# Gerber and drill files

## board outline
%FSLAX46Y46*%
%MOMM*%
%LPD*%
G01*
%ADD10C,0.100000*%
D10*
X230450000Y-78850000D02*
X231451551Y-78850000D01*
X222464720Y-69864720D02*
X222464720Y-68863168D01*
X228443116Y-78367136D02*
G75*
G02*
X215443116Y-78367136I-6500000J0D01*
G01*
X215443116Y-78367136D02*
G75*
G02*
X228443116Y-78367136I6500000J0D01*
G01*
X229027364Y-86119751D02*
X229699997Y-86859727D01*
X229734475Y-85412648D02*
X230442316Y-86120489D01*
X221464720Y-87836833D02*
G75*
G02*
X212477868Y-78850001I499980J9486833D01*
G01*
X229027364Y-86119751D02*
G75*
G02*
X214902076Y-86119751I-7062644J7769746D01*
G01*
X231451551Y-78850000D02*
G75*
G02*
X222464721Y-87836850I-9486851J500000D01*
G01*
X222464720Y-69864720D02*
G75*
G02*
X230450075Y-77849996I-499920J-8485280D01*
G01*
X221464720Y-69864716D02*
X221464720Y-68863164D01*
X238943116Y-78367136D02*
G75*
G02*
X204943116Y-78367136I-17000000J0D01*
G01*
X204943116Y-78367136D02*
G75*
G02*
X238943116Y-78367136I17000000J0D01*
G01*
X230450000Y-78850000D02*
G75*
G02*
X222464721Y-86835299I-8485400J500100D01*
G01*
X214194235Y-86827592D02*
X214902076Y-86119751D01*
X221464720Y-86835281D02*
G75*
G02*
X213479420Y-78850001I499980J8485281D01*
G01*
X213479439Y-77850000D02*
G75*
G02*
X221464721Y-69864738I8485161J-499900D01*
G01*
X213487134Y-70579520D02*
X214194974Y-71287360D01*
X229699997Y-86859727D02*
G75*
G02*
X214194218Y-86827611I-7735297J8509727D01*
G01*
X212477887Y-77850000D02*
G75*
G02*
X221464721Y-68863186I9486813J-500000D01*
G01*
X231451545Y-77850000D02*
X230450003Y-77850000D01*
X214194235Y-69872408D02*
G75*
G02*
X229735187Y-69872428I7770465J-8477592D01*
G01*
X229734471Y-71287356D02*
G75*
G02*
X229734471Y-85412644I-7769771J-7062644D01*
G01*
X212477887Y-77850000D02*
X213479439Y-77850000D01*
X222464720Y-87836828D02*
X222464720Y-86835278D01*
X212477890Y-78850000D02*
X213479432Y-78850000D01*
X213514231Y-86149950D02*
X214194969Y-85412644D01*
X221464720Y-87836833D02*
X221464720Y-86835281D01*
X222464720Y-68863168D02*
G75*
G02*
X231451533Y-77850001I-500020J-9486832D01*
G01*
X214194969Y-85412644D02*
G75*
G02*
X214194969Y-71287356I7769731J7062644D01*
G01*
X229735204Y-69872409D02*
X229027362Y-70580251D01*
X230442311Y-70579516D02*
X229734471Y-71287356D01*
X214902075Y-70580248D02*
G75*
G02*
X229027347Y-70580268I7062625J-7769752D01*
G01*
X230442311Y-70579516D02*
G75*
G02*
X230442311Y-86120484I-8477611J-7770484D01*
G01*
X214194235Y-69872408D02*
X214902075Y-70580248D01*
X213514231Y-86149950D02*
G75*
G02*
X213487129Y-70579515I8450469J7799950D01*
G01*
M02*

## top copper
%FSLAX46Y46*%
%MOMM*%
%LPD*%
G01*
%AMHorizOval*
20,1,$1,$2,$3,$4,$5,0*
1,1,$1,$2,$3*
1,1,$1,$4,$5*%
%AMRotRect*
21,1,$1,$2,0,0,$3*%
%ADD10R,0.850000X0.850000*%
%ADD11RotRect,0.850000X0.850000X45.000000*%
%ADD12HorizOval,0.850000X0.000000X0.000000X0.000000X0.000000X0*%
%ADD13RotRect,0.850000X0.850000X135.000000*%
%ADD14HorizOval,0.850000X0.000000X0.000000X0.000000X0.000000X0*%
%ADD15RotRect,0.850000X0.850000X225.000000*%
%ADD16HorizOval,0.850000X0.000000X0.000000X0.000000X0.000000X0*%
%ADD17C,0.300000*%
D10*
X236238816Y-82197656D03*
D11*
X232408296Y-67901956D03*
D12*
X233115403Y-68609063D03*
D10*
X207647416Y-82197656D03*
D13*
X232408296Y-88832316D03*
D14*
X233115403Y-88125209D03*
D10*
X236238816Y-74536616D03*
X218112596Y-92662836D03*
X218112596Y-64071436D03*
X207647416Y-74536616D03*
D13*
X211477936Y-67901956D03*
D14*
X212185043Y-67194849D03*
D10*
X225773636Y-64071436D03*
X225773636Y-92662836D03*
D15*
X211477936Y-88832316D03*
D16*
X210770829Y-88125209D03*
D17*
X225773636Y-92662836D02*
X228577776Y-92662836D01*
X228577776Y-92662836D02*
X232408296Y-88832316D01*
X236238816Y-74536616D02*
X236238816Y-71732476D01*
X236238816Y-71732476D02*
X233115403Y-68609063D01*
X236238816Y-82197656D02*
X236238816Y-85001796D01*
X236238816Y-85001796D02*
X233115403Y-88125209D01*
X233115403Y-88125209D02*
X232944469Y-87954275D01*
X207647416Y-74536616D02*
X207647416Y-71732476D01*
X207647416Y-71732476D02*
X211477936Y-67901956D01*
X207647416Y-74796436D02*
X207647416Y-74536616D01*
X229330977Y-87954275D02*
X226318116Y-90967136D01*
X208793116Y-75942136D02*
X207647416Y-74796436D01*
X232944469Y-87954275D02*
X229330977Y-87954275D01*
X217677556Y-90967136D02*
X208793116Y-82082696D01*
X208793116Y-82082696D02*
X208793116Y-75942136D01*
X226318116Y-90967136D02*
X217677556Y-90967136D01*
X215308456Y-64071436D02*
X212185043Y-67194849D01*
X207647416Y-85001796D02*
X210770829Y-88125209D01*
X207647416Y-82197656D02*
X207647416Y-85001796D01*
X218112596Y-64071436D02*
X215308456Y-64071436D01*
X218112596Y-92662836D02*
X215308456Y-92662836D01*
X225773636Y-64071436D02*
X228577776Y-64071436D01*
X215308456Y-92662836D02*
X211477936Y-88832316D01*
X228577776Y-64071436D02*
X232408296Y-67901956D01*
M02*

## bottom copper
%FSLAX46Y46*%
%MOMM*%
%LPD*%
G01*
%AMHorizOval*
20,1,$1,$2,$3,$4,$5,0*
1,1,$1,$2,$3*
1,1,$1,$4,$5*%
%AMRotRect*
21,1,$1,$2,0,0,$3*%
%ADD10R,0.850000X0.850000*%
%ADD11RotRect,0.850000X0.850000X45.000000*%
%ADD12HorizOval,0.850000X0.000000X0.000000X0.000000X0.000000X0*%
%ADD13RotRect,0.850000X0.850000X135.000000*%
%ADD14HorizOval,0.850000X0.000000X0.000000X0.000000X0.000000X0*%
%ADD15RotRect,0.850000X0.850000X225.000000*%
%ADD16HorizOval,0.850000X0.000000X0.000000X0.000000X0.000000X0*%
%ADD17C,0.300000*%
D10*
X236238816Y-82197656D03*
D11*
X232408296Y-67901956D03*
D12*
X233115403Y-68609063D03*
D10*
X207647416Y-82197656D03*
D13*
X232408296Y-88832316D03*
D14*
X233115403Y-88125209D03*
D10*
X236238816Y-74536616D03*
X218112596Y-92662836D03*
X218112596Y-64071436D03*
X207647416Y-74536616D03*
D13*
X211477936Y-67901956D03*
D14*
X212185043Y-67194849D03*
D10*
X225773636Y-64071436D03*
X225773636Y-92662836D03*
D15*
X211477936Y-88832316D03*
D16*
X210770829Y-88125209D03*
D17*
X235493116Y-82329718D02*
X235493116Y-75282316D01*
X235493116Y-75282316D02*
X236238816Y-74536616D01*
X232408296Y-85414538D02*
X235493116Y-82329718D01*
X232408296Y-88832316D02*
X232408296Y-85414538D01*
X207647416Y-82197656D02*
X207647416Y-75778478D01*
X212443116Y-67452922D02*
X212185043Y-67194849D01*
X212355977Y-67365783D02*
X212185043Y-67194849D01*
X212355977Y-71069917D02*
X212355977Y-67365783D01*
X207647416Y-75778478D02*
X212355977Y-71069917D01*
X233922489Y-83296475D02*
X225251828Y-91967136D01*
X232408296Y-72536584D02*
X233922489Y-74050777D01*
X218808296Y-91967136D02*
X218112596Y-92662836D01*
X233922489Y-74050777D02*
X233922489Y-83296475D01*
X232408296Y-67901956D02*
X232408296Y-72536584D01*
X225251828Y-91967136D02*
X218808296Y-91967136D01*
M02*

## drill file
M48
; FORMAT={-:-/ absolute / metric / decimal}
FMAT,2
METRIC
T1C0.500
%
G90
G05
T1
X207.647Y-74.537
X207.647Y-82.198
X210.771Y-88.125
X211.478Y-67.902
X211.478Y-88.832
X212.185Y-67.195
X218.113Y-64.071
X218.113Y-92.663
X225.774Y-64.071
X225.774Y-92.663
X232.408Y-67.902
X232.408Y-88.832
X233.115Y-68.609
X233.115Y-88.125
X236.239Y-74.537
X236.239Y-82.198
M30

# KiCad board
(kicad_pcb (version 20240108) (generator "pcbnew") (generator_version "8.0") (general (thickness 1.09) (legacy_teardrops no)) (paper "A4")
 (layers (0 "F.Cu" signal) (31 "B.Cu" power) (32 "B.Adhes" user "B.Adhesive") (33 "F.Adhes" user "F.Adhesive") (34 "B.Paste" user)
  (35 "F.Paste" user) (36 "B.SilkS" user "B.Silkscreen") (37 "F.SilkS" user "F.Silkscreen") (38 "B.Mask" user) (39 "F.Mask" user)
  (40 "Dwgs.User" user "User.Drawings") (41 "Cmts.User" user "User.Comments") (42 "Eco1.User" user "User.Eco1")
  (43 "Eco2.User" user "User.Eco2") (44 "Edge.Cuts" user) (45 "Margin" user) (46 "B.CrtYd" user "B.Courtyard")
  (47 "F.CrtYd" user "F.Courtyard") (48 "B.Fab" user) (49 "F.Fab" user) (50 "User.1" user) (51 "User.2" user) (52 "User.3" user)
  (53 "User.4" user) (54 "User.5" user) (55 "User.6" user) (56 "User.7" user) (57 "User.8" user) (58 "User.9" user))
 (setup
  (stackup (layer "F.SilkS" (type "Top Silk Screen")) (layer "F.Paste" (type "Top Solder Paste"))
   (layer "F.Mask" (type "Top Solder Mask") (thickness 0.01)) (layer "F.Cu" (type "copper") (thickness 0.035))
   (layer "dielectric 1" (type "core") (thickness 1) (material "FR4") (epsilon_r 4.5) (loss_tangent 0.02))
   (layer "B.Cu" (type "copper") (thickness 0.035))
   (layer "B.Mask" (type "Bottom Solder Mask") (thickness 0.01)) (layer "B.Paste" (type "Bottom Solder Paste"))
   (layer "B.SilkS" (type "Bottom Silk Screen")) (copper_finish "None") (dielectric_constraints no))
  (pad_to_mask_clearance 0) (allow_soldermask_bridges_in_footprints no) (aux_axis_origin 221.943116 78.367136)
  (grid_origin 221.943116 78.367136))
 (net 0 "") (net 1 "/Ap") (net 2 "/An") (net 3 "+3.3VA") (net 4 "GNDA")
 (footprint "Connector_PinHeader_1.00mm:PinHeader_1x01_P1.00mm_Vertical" (layer "F.Cu") (at 236.238816 82.197656)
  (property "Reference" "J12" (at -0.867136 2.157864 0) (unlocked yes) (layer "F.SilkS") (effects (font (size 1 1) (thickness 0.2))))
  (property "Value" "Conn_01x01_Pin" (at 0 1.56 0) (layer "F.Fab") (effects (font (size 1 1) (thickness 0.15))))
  (pad "1" thru_hole rect (at 0 0) (size 0.85 0.85) (drill 0.5) (layers "*.Cu" "*.Mask") (remove_unused_layers no) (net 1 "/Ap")))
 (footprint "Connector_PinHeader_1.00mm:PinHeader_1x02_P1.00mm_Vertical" (layer "F.Cu") (at 232.408296 67.901956 45)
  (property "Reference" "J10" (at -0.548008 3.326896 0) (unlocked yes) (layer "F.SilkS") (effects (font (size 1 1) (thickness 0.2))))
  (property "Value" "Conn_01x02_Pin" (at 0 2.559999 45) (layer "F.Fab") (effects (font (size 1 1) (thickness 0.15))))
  (pad "1" thru_hole rect (at 0 0 45) (size 0.85 0.85) (drill 0.5) (layers "*.Cu" "*.Mask") (remove_unused_layers no) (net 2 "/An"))
  (pad "2" thru_hole oval (at 0 1 45) (size 0.85 0.85) (drill 0.5) (layers "*.Cu" "*.Mask") (remove_unused_layers no) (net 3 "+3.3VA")))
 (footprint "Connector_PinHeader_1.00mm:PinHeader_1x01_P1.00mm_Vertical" (layer "F.Cu") (at 207.647416 82.197656)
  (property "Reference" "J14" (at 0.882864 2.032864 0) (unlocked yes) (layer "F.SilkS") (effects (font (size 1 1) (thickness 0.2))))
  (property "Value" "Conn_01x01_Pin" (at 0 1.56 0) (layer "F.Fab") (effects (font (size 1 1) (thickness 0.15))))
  (pad "1" thru_hole rect (at 0 0) (size 0.85 0.85) (drill 0.5) (layers "*.Cu" "*.Mask") (remove_unused_layers no) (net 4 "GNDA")))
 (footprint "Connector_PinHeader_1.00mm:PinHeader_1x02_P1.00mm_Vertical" (layer "F.Cu") (at 232.408296 88.832316 135)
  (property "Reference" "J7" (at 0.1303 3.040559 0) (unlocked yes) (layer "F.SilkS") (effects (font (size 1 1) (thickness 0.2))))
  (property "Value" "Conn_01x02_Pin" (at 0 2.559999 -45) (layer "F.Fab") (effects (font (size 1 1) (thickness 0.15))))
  (pad "1" thru_hole rect (at 0 0 135) (size 0.85 0.85) (drill 0.5) (layers "*.Cu" "*.Mask") (remove_unused_layers no) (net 3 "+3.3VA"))
  (pad "2" thru_hole oval (at 0 1 135) (size 0.85 0.85) (drill 0.5) (layers "*.Cu" "*.Mask") (remove_unused_layers no) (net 1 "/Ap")))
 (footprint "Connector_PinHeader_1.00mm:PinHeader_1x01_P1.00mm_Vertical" (layer "F.Cu") (at 236.238816 74.536616)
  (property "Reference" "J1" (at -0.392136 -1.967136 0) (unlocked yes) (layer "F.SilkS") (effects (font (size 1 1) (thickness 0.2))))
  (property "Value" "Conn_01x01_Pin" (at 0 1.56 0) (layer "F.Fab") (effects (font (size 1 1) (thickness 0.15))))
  (pad "1" thru_hole rect (at 0 0) (size 0.85 0.85) (drill 0.5) (layers "*.Cu" "*.Mask") (remove_unused_layers no) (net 3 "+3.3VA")))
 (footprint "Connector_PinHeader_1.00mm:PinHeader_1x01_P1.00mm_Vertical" (layer "F.Cu") (at 218.112596 92.662836)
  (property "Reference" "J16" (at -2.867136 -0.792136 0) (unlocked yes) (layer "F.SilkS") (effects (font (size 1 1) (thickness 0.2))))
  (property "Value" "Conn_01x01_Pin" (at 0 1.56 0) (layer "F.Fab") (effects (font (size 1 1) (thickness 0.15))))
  (pad "1" thru_hole rect (at 0 0) (size 0.85 0.85) (drill 0.5) (layers "*.Cu" "*.Mask") (remove_unused_layers no) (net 2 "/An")))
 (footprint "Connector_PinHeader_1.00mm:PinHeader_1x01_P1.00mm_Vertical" (layer "F.Cu") (at 218.112596 64.071436)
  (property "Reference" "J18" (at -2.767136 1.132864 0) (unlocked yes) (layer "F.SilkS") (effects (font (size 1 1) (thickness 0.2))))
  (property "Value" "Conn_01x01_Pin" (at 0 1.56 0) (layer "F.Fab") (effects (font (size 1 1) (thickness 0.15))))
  (pad "1" thru_hole rect (at 0 0) (size 0.85 0.85) (drill 0.5) (layers "*.Cu" "*.Mask") (remove_unused_layers no) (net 4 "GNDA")))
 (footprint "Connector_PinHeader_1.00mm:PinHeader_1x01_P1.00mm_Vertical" (layer "F.Cu") (at 207.647416 74.536616)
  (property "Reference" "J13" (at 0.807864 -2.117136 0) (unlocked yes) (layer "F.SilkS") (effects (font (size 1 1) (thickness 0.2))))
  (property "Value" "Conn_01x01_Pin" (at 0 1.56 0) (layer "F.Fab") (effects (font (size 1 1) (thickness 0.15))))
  (pad "1" thru_hole rect (at 0 0) (size 0.85 0.85) (drill 0.5) (layers "*.Cu" "*.Mask") (remove_unused_layers no) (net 1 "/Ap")))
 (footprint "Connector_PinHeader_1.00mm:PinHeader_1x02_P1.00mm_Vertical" (layer "F.Cu") (at 211.477936 67.901956 135)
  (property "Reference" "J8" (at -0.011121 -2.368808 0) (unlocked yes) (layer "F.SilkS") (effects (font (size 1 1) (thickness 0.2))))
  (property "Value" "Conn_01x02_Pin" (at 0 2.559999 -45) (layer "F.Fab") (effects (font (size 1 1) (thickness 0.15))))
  (pad "1" thru_hole rect (at 0 0 135) (size 0.85 0.85) (drill 0.5) (layers "*.Cu" "*.Mask") (remove_unused_layers no) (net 1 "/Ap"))
  (pad "2" thru_hole oval (at 0 1 135) (size 0.85 0.85) (drill 0.5) (layers "*.Cu" "*.Mask") (remove_unused_layers no) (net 4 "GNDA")))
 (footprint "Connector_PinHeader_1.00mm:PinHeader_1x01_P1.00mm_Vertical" (layer "F.Cu") (at 225.773636 64.071436)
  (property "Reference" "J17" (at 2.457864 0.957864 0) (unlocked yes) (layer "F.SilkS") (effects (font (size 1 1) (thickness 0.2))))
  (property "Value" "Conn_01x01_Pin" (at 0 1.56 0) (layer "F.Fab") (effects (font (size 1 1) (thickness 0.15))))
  (pad "1" thru_hole rect (at 0 0) (size 0.85 0.85) (drill 0.5) (layers "*.Cu" "*.Mask") (remove_unused_layers no) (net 2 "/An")))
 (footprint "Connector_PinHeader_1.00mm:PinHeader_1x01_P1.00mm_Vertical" (layer "F.Cu") (at 225.773636 92.662836)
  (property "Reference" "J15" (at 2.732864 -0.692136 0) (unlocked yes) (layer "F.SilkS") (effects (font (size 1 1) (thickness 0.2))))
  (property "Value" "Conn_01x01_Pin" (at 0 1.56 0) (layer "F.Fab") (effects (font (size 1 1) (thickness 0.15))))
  (pad "1" thru_hole rect (at 0 0) (size 0.85 0.85) (drill 0.5) (layers "*.Cu" "*.Mask") (remove_unused_layers no) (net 3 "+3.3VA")))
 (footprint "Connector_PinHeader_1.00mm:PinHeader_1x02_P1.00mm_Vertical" (layer "F.Cu") (at 211.477936 88.832316 -135)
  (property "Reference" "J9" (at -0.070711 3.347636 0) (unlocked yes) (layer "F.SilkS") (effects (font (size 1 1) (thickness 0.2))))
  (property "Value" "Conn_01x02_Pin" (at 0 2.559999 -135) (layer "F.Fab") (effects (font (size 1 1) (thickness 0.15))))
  (pad "1" thru_hole rect (at 0 0 225) (size 0.85 0.85) (drill 0.5) (layers "*.Cu" "*.Mask") (remove_unused_layers no) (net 2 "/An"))
  (pad "2" thru_hole oval (at 0 1 225) (size 0.85 0.85) (drill 0.5) (layers "*.Cu" "*.Mask") (remove_unused_layers no) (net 4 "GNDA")))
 (gr_line (start 230.45 78.85) (end 231.451551 78.85) (stroke (width 0.1) (type default)) (layer "Edge.Cuts"))
 (gr_line (start 222.46472 69.86472) (end 222.46472 68.863168) (stroke (width 0.1) (type default)) (layer "Edge.Cuts"))
 (gr_circle (center 221.943116 78.367136) (end 228.443116 78.367136) (stroke (width 0.1) (type default)) (fill none) (layer "Edge.Cuts"))
 (gr_line (start 229.027364 86.119751) (end 229.699997 86.859727) (stroke (width 0.1) (type default)) (layer "Edge.Cuts"))
 (gr_line (start 229.734475 85.412648) (end 230.442316 86.120489) (stroke (width 0.1) (type default)) (layer "Edge.Cuts"))
 (gr_arc (start 221.46472 87.836833) (mid 215.247206 85.067515) (end 212.47789 78.85) (stroke (width 0.1) (type default))
  (layer "Edge.Cuts"))
 (gr_arc (start 229.027364 86.119751) (mid 221.96472 88.85) (end 214.902076 86.119751) (stroke (width 0.1) (type default))
  (layer "Edge.Cuts"))
 (gr_arc (start 231.451551 78.85) (mid 228.682237 85.067516) (end 222.46472 87.836828) (stroke (width 0.1) (type default))
  (layer "Edge.Cuts"))
 (gr_arc (start 222.46472 69.86472) (mid 227.975137 72.339584) (end 230.450003 77.85) (stroke (width 0.1) (type default))
  (layer "Edge.Cuts"))
 (gr_line (start 221.46472 69.864716) (end 221.46472 68.863164) (stroke (width 0.1) (type default)) (layer "Edge.Cuts"))
 (gr_circle (center 221.943116 78.367136) (end 238.943116 78.367136) (stroke (width 0.1) (type default)) (fill none) (layer "Edge.Cuts"))
 (gr_arc (start 230.45 78.85) (mid 227.975105 84.360384) (end 222.46472 86.835278) (stroke (width 0.1) (type default)) (layer "Edge.Cuts"))
 (gr_line (start 214.194235 86.827592) (end 214.902076 86.119751) (stroke (width 0.1) (type default)) (layer "Edge.Cuts"))
 (gr_arc (start 221.46472 86.835281) (mid 215.95431 84.360408) (end 213.479432 78.85) (stroke (width 0.1) (type default))
  (layer "Edge.Cuts"))
 (gr_arc (start 213.479439 77.85) (mid 215.954288 72.339568) (end 221.46472 69.864716) (stroke (width 0.1) (type default))
  (layer "Edge.Cuts"))
 (gr_line (start 213.487134 70.57952) (end 214.194974 71.28736) (stroke (width 0.1) (type default)) (layer "Edge.Cuts"))
 (gr_arc (start 229.699997 86.859727) (mid 221.940886 89.849979) (end 214.194235 86.827592) (stroke (width 0.1) (type default))
  (layer "Edge.Cuts"))
 (gr_arc (start 212.477887 77.85) (mid 215.247209 71.632488) (end 221.46472 68.863164) (stroke (width 0.1) (type default))
  (layer "Edge.Cuts"))
 (gr_line (start 231.451545 77.85) (end 230.450003 77.85) (stroke (width 0.1) (type default)) (layer "Edge.Cuts"))
 (gr_arc (start 214.194235 69.872408) (mid 221.96472 66.85) (end 229.735204 69.872409) (stroke (width 0.1) (type default))
  (layer "Edge.Cuts"))
 (gr_arc (start 229.734471 71.287356) (mid 232.464724 78.350001) (end 229.734475 85.412648) (stroke (width 0.1) (type default))
  (layer "Edge.Cuts"))
 (gr_line (start 212.477887 77.85) (end 213.479439 77.85) (stroke (width 0.1) (type default)) (layer "Edge.Cuts"))
 (gr_line (start 222.46472 87.836828) (end 222.46472 86.835278) (stroke (width 0.1) (type default)) (layer "Edge.Cuts"))
 (gr_line (start 212.47789 78.85) (end 213.479432 78.85) (stroke (width 0.1) (type default)) (layer "Edge.Cuts"))
 (gr_line (start 213.514231 86.14995) (end 214.194969 85.412644) (stroke (width 0.1) (type default)) (layer "Edge.Cuts"))
 (gr_line (start 221.46472 87.836833) (end 221.46472 86.835281) (stroke (width 0.1) (type default)) (layer "Edge.Cuts"))
 (gr_arc (start 222.46472 68.863168) (mid 228.682231 71.632487) (end 231.451545 77.85) (stroke (width 0.1) (type default))
  (layer "Edge.Cuts"))
 (gr_arc (start 214.194969 85.412644) (mid 211.464724 78.350001) (end 214.194974 71.28736) (stroke (width 0.1) (type default))
  (layer "Edge.Cuts"))
 (gr_line (start 229.735204 69.872409) (end 229.027362 70.580251) (stroke (width 0.1) (type default)) (layer "Edge.Cuts"))
 (gr_line (start 230.442311 70.579516) (end 229.734471 71.287356) (stroke (width 0.1) (type default)) (layer "Edge.Cuts"))
 (gr_arc (start 214.902075 70.580248) (mid 221.964719 67.85) (end 229.027362 70.580251) (stroke (width 0.1) (type default))
  (layer "Edge.Cuts"))
 (gr_arc (start 230.442311 70.579516) (mid 233.464722 78.350001) (end 230.442316 86.120489) (stroke (width 0.1) (type default))
  (layer "Edge.Cuts"))
 (gr_line (start 214.194235 69.872408) (end 214.902075 70.580248) (stroke (width 0.1) (type default)) (layer "Edge.Cuts"))
 (gr_arc (start 213.514231 86.14995) (mid 210.464741 78.370018) (end 213.487134 70.57952) (stroke (width 0.1) (type default))
  (layer "Edge.Cuts"))
 (segment (start 225.773636 92.662836) (end 228.577776 92.662836) (width 0.3) (layer "F.Cu") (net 3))
 (segment (start 228.577776 92.662836) (end 232.408296 88.832316) (width 0.3) (layer "F.Cu") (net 3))
 (segment (start 236.238816 74.536616) (end 236.238816 71.732476) (width 0.3) (layer "F.Cu") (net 3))
 (segment (start 236.238816 71.732476) (end 233.115403 68.609063) (width 0.3) (layer "F.Cu") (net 3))
 (segment (start 235.493116 82.329718) (end 235.493116 75.282316) (width 0.3) (layer "B.Cu") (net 3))
 (segment (start 235.493116 75.282316) (end 236.238816 74.536616) (width 0.3) (layer "B.Cu") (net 3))
 (segment (start 232.408296 85.414538) (end 235.493116 82.329718) (width 0.3) (layer "B.Cu") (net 3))
 (segment (start 232.408296 88.832316) (end 232.408296 85.414538) (width 0.3) (layer "B.Cu") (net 3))
 (segment (start 236.238816 82.197656) (end 236.238816 85.001796) (width 0.3) (layer "F.Cu") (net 1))
 (segment (start 236.238816 85.001796) (end 233.115403 88.125209) (width 0.3) (layer "F.Cu") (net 1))
 (segment (start 233.115403 88.125209) (end 232.944469 87.954275) (width 0.3) (layer "F.Cu") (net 1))
 (segment (start 207.647416 74.536616) (end 207.647416 71.732476) (width 0.3) (layer "F.Cu") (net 1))
 (segment (start 207.647416 71.732476) (end 211.477936 67.901956) (width 0.3) (layer "F.Cu") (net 1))
 (segment (start 207.647416 74.796436) (end 207.647416 74.536616) (width 0.3) (layer "F.Cu") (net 1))
 (segment (start 229.330977 87.954275) (end 226.318116 90.967136) (width 0.3) (layer "F.Cu") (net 1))
 (segment (start 208.793116 75.942136) (end 207.647416 74.796436) (width 0.3) (layer "F.Cu") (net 1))
 (segment (start 232.944469 87.954275) (end 229.330977 87.954275) (width 0.3) (layer "F.Cu") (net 1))
 (segment (start 217.677556 90.967136) (end 208.793116 82.082696) (width 0.3) (layer "F.Cu") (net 1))
 (segment (start 208.793116 82.082696) (end 208.793116 75.942136) (width 0.3) (layer "F.Cu") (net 1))
 (segment (start 226.318116 90.967136) (end 217.677556 90.967136) (width 0.3) (layer "F.Cu") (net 1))
 (segment (start 215.308456 64.071436) (end 212.185043 67.194849) (width 0.3) (layer "F.Cu") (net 4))
 (segment (start 207.647416 85.001796) (end 210.770829 88.125209) (width 0.3) (layer "F.Cu") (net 4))
 (segment (start 207.647416 82.197656) (end 207.647416 85.001796) (width 0.3) (layer "F.Cu") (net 4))
 (segment (start 218.112596 64.071436) (end 215.308456 64.071436) (width 0.3) (layer "F.Cu") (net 4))
 (segment (start 207.647416 82.197656) (end 207.647416 75.778478) (width 0.3) (layer "B.Cu") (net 4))
 (segment (start 212.443116 67.452922) (end 212.185043 67.194849) (width 0.3) (layer "B.Cu") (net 4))
 (segment (start 212.355977 67.365783) (end 212.185043 67.194849) (width 0.3) (layer "B.Cu") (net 4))
 (segment (start 212.355977 71.069917) (end 212.355977 67.365783) (width 0.3) (layer "B.Cu") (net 4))
 (segment (start 207.647416 75.778478) (end 212.355977 71.069917) (width 0.3) (layer "B.Cu") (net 4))
 (segment (start 218.112596 92.662836) (end 215.308456 92.662836) (width 0.3) (layer "F.Cu") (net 2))
 (segment (start 225.773636 64.071436) (end 228.577776 64.071436) (width 0.3) (layer "F.Cu") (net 2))
 (segment (start 215.308456 92.662836) (end 211.477936 88.832316) (width 0.3) (layer "F.Cu") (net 2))
 (segment (start 228.577776 64.071436) (end 232.408296 67.901956) (width 0.3) (layer "F.Cu") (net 2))
 (segment (start 233.922489 83.296475) (end 225.251828 91.967136) (width 0.3) (layer "B.Cu") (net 2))
 (segment (start 232.408296 72.536584) (end 233.922489 74.050777) (width 0.3) (layer "B.Cu") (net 2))
 (segment (start 218.808296 91.967136) (end 218.112596 92.662836) (width 0.3) (layer "B.Cu") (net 2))
 (segment (start 233.922489 74.050777) (end 233.922489 83.296475) (width 0.3) (layer "B.Cu") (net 2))
 (segment (start 232.408296 67.901956) (end 232.408296 72.536584) (width 0.3) (layer "B.Cu") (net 2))
 (segment (start 225.251828 91.967136) (end 218.808296 91.967136) (width 0.3) (layer "B.Cu") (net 2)))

